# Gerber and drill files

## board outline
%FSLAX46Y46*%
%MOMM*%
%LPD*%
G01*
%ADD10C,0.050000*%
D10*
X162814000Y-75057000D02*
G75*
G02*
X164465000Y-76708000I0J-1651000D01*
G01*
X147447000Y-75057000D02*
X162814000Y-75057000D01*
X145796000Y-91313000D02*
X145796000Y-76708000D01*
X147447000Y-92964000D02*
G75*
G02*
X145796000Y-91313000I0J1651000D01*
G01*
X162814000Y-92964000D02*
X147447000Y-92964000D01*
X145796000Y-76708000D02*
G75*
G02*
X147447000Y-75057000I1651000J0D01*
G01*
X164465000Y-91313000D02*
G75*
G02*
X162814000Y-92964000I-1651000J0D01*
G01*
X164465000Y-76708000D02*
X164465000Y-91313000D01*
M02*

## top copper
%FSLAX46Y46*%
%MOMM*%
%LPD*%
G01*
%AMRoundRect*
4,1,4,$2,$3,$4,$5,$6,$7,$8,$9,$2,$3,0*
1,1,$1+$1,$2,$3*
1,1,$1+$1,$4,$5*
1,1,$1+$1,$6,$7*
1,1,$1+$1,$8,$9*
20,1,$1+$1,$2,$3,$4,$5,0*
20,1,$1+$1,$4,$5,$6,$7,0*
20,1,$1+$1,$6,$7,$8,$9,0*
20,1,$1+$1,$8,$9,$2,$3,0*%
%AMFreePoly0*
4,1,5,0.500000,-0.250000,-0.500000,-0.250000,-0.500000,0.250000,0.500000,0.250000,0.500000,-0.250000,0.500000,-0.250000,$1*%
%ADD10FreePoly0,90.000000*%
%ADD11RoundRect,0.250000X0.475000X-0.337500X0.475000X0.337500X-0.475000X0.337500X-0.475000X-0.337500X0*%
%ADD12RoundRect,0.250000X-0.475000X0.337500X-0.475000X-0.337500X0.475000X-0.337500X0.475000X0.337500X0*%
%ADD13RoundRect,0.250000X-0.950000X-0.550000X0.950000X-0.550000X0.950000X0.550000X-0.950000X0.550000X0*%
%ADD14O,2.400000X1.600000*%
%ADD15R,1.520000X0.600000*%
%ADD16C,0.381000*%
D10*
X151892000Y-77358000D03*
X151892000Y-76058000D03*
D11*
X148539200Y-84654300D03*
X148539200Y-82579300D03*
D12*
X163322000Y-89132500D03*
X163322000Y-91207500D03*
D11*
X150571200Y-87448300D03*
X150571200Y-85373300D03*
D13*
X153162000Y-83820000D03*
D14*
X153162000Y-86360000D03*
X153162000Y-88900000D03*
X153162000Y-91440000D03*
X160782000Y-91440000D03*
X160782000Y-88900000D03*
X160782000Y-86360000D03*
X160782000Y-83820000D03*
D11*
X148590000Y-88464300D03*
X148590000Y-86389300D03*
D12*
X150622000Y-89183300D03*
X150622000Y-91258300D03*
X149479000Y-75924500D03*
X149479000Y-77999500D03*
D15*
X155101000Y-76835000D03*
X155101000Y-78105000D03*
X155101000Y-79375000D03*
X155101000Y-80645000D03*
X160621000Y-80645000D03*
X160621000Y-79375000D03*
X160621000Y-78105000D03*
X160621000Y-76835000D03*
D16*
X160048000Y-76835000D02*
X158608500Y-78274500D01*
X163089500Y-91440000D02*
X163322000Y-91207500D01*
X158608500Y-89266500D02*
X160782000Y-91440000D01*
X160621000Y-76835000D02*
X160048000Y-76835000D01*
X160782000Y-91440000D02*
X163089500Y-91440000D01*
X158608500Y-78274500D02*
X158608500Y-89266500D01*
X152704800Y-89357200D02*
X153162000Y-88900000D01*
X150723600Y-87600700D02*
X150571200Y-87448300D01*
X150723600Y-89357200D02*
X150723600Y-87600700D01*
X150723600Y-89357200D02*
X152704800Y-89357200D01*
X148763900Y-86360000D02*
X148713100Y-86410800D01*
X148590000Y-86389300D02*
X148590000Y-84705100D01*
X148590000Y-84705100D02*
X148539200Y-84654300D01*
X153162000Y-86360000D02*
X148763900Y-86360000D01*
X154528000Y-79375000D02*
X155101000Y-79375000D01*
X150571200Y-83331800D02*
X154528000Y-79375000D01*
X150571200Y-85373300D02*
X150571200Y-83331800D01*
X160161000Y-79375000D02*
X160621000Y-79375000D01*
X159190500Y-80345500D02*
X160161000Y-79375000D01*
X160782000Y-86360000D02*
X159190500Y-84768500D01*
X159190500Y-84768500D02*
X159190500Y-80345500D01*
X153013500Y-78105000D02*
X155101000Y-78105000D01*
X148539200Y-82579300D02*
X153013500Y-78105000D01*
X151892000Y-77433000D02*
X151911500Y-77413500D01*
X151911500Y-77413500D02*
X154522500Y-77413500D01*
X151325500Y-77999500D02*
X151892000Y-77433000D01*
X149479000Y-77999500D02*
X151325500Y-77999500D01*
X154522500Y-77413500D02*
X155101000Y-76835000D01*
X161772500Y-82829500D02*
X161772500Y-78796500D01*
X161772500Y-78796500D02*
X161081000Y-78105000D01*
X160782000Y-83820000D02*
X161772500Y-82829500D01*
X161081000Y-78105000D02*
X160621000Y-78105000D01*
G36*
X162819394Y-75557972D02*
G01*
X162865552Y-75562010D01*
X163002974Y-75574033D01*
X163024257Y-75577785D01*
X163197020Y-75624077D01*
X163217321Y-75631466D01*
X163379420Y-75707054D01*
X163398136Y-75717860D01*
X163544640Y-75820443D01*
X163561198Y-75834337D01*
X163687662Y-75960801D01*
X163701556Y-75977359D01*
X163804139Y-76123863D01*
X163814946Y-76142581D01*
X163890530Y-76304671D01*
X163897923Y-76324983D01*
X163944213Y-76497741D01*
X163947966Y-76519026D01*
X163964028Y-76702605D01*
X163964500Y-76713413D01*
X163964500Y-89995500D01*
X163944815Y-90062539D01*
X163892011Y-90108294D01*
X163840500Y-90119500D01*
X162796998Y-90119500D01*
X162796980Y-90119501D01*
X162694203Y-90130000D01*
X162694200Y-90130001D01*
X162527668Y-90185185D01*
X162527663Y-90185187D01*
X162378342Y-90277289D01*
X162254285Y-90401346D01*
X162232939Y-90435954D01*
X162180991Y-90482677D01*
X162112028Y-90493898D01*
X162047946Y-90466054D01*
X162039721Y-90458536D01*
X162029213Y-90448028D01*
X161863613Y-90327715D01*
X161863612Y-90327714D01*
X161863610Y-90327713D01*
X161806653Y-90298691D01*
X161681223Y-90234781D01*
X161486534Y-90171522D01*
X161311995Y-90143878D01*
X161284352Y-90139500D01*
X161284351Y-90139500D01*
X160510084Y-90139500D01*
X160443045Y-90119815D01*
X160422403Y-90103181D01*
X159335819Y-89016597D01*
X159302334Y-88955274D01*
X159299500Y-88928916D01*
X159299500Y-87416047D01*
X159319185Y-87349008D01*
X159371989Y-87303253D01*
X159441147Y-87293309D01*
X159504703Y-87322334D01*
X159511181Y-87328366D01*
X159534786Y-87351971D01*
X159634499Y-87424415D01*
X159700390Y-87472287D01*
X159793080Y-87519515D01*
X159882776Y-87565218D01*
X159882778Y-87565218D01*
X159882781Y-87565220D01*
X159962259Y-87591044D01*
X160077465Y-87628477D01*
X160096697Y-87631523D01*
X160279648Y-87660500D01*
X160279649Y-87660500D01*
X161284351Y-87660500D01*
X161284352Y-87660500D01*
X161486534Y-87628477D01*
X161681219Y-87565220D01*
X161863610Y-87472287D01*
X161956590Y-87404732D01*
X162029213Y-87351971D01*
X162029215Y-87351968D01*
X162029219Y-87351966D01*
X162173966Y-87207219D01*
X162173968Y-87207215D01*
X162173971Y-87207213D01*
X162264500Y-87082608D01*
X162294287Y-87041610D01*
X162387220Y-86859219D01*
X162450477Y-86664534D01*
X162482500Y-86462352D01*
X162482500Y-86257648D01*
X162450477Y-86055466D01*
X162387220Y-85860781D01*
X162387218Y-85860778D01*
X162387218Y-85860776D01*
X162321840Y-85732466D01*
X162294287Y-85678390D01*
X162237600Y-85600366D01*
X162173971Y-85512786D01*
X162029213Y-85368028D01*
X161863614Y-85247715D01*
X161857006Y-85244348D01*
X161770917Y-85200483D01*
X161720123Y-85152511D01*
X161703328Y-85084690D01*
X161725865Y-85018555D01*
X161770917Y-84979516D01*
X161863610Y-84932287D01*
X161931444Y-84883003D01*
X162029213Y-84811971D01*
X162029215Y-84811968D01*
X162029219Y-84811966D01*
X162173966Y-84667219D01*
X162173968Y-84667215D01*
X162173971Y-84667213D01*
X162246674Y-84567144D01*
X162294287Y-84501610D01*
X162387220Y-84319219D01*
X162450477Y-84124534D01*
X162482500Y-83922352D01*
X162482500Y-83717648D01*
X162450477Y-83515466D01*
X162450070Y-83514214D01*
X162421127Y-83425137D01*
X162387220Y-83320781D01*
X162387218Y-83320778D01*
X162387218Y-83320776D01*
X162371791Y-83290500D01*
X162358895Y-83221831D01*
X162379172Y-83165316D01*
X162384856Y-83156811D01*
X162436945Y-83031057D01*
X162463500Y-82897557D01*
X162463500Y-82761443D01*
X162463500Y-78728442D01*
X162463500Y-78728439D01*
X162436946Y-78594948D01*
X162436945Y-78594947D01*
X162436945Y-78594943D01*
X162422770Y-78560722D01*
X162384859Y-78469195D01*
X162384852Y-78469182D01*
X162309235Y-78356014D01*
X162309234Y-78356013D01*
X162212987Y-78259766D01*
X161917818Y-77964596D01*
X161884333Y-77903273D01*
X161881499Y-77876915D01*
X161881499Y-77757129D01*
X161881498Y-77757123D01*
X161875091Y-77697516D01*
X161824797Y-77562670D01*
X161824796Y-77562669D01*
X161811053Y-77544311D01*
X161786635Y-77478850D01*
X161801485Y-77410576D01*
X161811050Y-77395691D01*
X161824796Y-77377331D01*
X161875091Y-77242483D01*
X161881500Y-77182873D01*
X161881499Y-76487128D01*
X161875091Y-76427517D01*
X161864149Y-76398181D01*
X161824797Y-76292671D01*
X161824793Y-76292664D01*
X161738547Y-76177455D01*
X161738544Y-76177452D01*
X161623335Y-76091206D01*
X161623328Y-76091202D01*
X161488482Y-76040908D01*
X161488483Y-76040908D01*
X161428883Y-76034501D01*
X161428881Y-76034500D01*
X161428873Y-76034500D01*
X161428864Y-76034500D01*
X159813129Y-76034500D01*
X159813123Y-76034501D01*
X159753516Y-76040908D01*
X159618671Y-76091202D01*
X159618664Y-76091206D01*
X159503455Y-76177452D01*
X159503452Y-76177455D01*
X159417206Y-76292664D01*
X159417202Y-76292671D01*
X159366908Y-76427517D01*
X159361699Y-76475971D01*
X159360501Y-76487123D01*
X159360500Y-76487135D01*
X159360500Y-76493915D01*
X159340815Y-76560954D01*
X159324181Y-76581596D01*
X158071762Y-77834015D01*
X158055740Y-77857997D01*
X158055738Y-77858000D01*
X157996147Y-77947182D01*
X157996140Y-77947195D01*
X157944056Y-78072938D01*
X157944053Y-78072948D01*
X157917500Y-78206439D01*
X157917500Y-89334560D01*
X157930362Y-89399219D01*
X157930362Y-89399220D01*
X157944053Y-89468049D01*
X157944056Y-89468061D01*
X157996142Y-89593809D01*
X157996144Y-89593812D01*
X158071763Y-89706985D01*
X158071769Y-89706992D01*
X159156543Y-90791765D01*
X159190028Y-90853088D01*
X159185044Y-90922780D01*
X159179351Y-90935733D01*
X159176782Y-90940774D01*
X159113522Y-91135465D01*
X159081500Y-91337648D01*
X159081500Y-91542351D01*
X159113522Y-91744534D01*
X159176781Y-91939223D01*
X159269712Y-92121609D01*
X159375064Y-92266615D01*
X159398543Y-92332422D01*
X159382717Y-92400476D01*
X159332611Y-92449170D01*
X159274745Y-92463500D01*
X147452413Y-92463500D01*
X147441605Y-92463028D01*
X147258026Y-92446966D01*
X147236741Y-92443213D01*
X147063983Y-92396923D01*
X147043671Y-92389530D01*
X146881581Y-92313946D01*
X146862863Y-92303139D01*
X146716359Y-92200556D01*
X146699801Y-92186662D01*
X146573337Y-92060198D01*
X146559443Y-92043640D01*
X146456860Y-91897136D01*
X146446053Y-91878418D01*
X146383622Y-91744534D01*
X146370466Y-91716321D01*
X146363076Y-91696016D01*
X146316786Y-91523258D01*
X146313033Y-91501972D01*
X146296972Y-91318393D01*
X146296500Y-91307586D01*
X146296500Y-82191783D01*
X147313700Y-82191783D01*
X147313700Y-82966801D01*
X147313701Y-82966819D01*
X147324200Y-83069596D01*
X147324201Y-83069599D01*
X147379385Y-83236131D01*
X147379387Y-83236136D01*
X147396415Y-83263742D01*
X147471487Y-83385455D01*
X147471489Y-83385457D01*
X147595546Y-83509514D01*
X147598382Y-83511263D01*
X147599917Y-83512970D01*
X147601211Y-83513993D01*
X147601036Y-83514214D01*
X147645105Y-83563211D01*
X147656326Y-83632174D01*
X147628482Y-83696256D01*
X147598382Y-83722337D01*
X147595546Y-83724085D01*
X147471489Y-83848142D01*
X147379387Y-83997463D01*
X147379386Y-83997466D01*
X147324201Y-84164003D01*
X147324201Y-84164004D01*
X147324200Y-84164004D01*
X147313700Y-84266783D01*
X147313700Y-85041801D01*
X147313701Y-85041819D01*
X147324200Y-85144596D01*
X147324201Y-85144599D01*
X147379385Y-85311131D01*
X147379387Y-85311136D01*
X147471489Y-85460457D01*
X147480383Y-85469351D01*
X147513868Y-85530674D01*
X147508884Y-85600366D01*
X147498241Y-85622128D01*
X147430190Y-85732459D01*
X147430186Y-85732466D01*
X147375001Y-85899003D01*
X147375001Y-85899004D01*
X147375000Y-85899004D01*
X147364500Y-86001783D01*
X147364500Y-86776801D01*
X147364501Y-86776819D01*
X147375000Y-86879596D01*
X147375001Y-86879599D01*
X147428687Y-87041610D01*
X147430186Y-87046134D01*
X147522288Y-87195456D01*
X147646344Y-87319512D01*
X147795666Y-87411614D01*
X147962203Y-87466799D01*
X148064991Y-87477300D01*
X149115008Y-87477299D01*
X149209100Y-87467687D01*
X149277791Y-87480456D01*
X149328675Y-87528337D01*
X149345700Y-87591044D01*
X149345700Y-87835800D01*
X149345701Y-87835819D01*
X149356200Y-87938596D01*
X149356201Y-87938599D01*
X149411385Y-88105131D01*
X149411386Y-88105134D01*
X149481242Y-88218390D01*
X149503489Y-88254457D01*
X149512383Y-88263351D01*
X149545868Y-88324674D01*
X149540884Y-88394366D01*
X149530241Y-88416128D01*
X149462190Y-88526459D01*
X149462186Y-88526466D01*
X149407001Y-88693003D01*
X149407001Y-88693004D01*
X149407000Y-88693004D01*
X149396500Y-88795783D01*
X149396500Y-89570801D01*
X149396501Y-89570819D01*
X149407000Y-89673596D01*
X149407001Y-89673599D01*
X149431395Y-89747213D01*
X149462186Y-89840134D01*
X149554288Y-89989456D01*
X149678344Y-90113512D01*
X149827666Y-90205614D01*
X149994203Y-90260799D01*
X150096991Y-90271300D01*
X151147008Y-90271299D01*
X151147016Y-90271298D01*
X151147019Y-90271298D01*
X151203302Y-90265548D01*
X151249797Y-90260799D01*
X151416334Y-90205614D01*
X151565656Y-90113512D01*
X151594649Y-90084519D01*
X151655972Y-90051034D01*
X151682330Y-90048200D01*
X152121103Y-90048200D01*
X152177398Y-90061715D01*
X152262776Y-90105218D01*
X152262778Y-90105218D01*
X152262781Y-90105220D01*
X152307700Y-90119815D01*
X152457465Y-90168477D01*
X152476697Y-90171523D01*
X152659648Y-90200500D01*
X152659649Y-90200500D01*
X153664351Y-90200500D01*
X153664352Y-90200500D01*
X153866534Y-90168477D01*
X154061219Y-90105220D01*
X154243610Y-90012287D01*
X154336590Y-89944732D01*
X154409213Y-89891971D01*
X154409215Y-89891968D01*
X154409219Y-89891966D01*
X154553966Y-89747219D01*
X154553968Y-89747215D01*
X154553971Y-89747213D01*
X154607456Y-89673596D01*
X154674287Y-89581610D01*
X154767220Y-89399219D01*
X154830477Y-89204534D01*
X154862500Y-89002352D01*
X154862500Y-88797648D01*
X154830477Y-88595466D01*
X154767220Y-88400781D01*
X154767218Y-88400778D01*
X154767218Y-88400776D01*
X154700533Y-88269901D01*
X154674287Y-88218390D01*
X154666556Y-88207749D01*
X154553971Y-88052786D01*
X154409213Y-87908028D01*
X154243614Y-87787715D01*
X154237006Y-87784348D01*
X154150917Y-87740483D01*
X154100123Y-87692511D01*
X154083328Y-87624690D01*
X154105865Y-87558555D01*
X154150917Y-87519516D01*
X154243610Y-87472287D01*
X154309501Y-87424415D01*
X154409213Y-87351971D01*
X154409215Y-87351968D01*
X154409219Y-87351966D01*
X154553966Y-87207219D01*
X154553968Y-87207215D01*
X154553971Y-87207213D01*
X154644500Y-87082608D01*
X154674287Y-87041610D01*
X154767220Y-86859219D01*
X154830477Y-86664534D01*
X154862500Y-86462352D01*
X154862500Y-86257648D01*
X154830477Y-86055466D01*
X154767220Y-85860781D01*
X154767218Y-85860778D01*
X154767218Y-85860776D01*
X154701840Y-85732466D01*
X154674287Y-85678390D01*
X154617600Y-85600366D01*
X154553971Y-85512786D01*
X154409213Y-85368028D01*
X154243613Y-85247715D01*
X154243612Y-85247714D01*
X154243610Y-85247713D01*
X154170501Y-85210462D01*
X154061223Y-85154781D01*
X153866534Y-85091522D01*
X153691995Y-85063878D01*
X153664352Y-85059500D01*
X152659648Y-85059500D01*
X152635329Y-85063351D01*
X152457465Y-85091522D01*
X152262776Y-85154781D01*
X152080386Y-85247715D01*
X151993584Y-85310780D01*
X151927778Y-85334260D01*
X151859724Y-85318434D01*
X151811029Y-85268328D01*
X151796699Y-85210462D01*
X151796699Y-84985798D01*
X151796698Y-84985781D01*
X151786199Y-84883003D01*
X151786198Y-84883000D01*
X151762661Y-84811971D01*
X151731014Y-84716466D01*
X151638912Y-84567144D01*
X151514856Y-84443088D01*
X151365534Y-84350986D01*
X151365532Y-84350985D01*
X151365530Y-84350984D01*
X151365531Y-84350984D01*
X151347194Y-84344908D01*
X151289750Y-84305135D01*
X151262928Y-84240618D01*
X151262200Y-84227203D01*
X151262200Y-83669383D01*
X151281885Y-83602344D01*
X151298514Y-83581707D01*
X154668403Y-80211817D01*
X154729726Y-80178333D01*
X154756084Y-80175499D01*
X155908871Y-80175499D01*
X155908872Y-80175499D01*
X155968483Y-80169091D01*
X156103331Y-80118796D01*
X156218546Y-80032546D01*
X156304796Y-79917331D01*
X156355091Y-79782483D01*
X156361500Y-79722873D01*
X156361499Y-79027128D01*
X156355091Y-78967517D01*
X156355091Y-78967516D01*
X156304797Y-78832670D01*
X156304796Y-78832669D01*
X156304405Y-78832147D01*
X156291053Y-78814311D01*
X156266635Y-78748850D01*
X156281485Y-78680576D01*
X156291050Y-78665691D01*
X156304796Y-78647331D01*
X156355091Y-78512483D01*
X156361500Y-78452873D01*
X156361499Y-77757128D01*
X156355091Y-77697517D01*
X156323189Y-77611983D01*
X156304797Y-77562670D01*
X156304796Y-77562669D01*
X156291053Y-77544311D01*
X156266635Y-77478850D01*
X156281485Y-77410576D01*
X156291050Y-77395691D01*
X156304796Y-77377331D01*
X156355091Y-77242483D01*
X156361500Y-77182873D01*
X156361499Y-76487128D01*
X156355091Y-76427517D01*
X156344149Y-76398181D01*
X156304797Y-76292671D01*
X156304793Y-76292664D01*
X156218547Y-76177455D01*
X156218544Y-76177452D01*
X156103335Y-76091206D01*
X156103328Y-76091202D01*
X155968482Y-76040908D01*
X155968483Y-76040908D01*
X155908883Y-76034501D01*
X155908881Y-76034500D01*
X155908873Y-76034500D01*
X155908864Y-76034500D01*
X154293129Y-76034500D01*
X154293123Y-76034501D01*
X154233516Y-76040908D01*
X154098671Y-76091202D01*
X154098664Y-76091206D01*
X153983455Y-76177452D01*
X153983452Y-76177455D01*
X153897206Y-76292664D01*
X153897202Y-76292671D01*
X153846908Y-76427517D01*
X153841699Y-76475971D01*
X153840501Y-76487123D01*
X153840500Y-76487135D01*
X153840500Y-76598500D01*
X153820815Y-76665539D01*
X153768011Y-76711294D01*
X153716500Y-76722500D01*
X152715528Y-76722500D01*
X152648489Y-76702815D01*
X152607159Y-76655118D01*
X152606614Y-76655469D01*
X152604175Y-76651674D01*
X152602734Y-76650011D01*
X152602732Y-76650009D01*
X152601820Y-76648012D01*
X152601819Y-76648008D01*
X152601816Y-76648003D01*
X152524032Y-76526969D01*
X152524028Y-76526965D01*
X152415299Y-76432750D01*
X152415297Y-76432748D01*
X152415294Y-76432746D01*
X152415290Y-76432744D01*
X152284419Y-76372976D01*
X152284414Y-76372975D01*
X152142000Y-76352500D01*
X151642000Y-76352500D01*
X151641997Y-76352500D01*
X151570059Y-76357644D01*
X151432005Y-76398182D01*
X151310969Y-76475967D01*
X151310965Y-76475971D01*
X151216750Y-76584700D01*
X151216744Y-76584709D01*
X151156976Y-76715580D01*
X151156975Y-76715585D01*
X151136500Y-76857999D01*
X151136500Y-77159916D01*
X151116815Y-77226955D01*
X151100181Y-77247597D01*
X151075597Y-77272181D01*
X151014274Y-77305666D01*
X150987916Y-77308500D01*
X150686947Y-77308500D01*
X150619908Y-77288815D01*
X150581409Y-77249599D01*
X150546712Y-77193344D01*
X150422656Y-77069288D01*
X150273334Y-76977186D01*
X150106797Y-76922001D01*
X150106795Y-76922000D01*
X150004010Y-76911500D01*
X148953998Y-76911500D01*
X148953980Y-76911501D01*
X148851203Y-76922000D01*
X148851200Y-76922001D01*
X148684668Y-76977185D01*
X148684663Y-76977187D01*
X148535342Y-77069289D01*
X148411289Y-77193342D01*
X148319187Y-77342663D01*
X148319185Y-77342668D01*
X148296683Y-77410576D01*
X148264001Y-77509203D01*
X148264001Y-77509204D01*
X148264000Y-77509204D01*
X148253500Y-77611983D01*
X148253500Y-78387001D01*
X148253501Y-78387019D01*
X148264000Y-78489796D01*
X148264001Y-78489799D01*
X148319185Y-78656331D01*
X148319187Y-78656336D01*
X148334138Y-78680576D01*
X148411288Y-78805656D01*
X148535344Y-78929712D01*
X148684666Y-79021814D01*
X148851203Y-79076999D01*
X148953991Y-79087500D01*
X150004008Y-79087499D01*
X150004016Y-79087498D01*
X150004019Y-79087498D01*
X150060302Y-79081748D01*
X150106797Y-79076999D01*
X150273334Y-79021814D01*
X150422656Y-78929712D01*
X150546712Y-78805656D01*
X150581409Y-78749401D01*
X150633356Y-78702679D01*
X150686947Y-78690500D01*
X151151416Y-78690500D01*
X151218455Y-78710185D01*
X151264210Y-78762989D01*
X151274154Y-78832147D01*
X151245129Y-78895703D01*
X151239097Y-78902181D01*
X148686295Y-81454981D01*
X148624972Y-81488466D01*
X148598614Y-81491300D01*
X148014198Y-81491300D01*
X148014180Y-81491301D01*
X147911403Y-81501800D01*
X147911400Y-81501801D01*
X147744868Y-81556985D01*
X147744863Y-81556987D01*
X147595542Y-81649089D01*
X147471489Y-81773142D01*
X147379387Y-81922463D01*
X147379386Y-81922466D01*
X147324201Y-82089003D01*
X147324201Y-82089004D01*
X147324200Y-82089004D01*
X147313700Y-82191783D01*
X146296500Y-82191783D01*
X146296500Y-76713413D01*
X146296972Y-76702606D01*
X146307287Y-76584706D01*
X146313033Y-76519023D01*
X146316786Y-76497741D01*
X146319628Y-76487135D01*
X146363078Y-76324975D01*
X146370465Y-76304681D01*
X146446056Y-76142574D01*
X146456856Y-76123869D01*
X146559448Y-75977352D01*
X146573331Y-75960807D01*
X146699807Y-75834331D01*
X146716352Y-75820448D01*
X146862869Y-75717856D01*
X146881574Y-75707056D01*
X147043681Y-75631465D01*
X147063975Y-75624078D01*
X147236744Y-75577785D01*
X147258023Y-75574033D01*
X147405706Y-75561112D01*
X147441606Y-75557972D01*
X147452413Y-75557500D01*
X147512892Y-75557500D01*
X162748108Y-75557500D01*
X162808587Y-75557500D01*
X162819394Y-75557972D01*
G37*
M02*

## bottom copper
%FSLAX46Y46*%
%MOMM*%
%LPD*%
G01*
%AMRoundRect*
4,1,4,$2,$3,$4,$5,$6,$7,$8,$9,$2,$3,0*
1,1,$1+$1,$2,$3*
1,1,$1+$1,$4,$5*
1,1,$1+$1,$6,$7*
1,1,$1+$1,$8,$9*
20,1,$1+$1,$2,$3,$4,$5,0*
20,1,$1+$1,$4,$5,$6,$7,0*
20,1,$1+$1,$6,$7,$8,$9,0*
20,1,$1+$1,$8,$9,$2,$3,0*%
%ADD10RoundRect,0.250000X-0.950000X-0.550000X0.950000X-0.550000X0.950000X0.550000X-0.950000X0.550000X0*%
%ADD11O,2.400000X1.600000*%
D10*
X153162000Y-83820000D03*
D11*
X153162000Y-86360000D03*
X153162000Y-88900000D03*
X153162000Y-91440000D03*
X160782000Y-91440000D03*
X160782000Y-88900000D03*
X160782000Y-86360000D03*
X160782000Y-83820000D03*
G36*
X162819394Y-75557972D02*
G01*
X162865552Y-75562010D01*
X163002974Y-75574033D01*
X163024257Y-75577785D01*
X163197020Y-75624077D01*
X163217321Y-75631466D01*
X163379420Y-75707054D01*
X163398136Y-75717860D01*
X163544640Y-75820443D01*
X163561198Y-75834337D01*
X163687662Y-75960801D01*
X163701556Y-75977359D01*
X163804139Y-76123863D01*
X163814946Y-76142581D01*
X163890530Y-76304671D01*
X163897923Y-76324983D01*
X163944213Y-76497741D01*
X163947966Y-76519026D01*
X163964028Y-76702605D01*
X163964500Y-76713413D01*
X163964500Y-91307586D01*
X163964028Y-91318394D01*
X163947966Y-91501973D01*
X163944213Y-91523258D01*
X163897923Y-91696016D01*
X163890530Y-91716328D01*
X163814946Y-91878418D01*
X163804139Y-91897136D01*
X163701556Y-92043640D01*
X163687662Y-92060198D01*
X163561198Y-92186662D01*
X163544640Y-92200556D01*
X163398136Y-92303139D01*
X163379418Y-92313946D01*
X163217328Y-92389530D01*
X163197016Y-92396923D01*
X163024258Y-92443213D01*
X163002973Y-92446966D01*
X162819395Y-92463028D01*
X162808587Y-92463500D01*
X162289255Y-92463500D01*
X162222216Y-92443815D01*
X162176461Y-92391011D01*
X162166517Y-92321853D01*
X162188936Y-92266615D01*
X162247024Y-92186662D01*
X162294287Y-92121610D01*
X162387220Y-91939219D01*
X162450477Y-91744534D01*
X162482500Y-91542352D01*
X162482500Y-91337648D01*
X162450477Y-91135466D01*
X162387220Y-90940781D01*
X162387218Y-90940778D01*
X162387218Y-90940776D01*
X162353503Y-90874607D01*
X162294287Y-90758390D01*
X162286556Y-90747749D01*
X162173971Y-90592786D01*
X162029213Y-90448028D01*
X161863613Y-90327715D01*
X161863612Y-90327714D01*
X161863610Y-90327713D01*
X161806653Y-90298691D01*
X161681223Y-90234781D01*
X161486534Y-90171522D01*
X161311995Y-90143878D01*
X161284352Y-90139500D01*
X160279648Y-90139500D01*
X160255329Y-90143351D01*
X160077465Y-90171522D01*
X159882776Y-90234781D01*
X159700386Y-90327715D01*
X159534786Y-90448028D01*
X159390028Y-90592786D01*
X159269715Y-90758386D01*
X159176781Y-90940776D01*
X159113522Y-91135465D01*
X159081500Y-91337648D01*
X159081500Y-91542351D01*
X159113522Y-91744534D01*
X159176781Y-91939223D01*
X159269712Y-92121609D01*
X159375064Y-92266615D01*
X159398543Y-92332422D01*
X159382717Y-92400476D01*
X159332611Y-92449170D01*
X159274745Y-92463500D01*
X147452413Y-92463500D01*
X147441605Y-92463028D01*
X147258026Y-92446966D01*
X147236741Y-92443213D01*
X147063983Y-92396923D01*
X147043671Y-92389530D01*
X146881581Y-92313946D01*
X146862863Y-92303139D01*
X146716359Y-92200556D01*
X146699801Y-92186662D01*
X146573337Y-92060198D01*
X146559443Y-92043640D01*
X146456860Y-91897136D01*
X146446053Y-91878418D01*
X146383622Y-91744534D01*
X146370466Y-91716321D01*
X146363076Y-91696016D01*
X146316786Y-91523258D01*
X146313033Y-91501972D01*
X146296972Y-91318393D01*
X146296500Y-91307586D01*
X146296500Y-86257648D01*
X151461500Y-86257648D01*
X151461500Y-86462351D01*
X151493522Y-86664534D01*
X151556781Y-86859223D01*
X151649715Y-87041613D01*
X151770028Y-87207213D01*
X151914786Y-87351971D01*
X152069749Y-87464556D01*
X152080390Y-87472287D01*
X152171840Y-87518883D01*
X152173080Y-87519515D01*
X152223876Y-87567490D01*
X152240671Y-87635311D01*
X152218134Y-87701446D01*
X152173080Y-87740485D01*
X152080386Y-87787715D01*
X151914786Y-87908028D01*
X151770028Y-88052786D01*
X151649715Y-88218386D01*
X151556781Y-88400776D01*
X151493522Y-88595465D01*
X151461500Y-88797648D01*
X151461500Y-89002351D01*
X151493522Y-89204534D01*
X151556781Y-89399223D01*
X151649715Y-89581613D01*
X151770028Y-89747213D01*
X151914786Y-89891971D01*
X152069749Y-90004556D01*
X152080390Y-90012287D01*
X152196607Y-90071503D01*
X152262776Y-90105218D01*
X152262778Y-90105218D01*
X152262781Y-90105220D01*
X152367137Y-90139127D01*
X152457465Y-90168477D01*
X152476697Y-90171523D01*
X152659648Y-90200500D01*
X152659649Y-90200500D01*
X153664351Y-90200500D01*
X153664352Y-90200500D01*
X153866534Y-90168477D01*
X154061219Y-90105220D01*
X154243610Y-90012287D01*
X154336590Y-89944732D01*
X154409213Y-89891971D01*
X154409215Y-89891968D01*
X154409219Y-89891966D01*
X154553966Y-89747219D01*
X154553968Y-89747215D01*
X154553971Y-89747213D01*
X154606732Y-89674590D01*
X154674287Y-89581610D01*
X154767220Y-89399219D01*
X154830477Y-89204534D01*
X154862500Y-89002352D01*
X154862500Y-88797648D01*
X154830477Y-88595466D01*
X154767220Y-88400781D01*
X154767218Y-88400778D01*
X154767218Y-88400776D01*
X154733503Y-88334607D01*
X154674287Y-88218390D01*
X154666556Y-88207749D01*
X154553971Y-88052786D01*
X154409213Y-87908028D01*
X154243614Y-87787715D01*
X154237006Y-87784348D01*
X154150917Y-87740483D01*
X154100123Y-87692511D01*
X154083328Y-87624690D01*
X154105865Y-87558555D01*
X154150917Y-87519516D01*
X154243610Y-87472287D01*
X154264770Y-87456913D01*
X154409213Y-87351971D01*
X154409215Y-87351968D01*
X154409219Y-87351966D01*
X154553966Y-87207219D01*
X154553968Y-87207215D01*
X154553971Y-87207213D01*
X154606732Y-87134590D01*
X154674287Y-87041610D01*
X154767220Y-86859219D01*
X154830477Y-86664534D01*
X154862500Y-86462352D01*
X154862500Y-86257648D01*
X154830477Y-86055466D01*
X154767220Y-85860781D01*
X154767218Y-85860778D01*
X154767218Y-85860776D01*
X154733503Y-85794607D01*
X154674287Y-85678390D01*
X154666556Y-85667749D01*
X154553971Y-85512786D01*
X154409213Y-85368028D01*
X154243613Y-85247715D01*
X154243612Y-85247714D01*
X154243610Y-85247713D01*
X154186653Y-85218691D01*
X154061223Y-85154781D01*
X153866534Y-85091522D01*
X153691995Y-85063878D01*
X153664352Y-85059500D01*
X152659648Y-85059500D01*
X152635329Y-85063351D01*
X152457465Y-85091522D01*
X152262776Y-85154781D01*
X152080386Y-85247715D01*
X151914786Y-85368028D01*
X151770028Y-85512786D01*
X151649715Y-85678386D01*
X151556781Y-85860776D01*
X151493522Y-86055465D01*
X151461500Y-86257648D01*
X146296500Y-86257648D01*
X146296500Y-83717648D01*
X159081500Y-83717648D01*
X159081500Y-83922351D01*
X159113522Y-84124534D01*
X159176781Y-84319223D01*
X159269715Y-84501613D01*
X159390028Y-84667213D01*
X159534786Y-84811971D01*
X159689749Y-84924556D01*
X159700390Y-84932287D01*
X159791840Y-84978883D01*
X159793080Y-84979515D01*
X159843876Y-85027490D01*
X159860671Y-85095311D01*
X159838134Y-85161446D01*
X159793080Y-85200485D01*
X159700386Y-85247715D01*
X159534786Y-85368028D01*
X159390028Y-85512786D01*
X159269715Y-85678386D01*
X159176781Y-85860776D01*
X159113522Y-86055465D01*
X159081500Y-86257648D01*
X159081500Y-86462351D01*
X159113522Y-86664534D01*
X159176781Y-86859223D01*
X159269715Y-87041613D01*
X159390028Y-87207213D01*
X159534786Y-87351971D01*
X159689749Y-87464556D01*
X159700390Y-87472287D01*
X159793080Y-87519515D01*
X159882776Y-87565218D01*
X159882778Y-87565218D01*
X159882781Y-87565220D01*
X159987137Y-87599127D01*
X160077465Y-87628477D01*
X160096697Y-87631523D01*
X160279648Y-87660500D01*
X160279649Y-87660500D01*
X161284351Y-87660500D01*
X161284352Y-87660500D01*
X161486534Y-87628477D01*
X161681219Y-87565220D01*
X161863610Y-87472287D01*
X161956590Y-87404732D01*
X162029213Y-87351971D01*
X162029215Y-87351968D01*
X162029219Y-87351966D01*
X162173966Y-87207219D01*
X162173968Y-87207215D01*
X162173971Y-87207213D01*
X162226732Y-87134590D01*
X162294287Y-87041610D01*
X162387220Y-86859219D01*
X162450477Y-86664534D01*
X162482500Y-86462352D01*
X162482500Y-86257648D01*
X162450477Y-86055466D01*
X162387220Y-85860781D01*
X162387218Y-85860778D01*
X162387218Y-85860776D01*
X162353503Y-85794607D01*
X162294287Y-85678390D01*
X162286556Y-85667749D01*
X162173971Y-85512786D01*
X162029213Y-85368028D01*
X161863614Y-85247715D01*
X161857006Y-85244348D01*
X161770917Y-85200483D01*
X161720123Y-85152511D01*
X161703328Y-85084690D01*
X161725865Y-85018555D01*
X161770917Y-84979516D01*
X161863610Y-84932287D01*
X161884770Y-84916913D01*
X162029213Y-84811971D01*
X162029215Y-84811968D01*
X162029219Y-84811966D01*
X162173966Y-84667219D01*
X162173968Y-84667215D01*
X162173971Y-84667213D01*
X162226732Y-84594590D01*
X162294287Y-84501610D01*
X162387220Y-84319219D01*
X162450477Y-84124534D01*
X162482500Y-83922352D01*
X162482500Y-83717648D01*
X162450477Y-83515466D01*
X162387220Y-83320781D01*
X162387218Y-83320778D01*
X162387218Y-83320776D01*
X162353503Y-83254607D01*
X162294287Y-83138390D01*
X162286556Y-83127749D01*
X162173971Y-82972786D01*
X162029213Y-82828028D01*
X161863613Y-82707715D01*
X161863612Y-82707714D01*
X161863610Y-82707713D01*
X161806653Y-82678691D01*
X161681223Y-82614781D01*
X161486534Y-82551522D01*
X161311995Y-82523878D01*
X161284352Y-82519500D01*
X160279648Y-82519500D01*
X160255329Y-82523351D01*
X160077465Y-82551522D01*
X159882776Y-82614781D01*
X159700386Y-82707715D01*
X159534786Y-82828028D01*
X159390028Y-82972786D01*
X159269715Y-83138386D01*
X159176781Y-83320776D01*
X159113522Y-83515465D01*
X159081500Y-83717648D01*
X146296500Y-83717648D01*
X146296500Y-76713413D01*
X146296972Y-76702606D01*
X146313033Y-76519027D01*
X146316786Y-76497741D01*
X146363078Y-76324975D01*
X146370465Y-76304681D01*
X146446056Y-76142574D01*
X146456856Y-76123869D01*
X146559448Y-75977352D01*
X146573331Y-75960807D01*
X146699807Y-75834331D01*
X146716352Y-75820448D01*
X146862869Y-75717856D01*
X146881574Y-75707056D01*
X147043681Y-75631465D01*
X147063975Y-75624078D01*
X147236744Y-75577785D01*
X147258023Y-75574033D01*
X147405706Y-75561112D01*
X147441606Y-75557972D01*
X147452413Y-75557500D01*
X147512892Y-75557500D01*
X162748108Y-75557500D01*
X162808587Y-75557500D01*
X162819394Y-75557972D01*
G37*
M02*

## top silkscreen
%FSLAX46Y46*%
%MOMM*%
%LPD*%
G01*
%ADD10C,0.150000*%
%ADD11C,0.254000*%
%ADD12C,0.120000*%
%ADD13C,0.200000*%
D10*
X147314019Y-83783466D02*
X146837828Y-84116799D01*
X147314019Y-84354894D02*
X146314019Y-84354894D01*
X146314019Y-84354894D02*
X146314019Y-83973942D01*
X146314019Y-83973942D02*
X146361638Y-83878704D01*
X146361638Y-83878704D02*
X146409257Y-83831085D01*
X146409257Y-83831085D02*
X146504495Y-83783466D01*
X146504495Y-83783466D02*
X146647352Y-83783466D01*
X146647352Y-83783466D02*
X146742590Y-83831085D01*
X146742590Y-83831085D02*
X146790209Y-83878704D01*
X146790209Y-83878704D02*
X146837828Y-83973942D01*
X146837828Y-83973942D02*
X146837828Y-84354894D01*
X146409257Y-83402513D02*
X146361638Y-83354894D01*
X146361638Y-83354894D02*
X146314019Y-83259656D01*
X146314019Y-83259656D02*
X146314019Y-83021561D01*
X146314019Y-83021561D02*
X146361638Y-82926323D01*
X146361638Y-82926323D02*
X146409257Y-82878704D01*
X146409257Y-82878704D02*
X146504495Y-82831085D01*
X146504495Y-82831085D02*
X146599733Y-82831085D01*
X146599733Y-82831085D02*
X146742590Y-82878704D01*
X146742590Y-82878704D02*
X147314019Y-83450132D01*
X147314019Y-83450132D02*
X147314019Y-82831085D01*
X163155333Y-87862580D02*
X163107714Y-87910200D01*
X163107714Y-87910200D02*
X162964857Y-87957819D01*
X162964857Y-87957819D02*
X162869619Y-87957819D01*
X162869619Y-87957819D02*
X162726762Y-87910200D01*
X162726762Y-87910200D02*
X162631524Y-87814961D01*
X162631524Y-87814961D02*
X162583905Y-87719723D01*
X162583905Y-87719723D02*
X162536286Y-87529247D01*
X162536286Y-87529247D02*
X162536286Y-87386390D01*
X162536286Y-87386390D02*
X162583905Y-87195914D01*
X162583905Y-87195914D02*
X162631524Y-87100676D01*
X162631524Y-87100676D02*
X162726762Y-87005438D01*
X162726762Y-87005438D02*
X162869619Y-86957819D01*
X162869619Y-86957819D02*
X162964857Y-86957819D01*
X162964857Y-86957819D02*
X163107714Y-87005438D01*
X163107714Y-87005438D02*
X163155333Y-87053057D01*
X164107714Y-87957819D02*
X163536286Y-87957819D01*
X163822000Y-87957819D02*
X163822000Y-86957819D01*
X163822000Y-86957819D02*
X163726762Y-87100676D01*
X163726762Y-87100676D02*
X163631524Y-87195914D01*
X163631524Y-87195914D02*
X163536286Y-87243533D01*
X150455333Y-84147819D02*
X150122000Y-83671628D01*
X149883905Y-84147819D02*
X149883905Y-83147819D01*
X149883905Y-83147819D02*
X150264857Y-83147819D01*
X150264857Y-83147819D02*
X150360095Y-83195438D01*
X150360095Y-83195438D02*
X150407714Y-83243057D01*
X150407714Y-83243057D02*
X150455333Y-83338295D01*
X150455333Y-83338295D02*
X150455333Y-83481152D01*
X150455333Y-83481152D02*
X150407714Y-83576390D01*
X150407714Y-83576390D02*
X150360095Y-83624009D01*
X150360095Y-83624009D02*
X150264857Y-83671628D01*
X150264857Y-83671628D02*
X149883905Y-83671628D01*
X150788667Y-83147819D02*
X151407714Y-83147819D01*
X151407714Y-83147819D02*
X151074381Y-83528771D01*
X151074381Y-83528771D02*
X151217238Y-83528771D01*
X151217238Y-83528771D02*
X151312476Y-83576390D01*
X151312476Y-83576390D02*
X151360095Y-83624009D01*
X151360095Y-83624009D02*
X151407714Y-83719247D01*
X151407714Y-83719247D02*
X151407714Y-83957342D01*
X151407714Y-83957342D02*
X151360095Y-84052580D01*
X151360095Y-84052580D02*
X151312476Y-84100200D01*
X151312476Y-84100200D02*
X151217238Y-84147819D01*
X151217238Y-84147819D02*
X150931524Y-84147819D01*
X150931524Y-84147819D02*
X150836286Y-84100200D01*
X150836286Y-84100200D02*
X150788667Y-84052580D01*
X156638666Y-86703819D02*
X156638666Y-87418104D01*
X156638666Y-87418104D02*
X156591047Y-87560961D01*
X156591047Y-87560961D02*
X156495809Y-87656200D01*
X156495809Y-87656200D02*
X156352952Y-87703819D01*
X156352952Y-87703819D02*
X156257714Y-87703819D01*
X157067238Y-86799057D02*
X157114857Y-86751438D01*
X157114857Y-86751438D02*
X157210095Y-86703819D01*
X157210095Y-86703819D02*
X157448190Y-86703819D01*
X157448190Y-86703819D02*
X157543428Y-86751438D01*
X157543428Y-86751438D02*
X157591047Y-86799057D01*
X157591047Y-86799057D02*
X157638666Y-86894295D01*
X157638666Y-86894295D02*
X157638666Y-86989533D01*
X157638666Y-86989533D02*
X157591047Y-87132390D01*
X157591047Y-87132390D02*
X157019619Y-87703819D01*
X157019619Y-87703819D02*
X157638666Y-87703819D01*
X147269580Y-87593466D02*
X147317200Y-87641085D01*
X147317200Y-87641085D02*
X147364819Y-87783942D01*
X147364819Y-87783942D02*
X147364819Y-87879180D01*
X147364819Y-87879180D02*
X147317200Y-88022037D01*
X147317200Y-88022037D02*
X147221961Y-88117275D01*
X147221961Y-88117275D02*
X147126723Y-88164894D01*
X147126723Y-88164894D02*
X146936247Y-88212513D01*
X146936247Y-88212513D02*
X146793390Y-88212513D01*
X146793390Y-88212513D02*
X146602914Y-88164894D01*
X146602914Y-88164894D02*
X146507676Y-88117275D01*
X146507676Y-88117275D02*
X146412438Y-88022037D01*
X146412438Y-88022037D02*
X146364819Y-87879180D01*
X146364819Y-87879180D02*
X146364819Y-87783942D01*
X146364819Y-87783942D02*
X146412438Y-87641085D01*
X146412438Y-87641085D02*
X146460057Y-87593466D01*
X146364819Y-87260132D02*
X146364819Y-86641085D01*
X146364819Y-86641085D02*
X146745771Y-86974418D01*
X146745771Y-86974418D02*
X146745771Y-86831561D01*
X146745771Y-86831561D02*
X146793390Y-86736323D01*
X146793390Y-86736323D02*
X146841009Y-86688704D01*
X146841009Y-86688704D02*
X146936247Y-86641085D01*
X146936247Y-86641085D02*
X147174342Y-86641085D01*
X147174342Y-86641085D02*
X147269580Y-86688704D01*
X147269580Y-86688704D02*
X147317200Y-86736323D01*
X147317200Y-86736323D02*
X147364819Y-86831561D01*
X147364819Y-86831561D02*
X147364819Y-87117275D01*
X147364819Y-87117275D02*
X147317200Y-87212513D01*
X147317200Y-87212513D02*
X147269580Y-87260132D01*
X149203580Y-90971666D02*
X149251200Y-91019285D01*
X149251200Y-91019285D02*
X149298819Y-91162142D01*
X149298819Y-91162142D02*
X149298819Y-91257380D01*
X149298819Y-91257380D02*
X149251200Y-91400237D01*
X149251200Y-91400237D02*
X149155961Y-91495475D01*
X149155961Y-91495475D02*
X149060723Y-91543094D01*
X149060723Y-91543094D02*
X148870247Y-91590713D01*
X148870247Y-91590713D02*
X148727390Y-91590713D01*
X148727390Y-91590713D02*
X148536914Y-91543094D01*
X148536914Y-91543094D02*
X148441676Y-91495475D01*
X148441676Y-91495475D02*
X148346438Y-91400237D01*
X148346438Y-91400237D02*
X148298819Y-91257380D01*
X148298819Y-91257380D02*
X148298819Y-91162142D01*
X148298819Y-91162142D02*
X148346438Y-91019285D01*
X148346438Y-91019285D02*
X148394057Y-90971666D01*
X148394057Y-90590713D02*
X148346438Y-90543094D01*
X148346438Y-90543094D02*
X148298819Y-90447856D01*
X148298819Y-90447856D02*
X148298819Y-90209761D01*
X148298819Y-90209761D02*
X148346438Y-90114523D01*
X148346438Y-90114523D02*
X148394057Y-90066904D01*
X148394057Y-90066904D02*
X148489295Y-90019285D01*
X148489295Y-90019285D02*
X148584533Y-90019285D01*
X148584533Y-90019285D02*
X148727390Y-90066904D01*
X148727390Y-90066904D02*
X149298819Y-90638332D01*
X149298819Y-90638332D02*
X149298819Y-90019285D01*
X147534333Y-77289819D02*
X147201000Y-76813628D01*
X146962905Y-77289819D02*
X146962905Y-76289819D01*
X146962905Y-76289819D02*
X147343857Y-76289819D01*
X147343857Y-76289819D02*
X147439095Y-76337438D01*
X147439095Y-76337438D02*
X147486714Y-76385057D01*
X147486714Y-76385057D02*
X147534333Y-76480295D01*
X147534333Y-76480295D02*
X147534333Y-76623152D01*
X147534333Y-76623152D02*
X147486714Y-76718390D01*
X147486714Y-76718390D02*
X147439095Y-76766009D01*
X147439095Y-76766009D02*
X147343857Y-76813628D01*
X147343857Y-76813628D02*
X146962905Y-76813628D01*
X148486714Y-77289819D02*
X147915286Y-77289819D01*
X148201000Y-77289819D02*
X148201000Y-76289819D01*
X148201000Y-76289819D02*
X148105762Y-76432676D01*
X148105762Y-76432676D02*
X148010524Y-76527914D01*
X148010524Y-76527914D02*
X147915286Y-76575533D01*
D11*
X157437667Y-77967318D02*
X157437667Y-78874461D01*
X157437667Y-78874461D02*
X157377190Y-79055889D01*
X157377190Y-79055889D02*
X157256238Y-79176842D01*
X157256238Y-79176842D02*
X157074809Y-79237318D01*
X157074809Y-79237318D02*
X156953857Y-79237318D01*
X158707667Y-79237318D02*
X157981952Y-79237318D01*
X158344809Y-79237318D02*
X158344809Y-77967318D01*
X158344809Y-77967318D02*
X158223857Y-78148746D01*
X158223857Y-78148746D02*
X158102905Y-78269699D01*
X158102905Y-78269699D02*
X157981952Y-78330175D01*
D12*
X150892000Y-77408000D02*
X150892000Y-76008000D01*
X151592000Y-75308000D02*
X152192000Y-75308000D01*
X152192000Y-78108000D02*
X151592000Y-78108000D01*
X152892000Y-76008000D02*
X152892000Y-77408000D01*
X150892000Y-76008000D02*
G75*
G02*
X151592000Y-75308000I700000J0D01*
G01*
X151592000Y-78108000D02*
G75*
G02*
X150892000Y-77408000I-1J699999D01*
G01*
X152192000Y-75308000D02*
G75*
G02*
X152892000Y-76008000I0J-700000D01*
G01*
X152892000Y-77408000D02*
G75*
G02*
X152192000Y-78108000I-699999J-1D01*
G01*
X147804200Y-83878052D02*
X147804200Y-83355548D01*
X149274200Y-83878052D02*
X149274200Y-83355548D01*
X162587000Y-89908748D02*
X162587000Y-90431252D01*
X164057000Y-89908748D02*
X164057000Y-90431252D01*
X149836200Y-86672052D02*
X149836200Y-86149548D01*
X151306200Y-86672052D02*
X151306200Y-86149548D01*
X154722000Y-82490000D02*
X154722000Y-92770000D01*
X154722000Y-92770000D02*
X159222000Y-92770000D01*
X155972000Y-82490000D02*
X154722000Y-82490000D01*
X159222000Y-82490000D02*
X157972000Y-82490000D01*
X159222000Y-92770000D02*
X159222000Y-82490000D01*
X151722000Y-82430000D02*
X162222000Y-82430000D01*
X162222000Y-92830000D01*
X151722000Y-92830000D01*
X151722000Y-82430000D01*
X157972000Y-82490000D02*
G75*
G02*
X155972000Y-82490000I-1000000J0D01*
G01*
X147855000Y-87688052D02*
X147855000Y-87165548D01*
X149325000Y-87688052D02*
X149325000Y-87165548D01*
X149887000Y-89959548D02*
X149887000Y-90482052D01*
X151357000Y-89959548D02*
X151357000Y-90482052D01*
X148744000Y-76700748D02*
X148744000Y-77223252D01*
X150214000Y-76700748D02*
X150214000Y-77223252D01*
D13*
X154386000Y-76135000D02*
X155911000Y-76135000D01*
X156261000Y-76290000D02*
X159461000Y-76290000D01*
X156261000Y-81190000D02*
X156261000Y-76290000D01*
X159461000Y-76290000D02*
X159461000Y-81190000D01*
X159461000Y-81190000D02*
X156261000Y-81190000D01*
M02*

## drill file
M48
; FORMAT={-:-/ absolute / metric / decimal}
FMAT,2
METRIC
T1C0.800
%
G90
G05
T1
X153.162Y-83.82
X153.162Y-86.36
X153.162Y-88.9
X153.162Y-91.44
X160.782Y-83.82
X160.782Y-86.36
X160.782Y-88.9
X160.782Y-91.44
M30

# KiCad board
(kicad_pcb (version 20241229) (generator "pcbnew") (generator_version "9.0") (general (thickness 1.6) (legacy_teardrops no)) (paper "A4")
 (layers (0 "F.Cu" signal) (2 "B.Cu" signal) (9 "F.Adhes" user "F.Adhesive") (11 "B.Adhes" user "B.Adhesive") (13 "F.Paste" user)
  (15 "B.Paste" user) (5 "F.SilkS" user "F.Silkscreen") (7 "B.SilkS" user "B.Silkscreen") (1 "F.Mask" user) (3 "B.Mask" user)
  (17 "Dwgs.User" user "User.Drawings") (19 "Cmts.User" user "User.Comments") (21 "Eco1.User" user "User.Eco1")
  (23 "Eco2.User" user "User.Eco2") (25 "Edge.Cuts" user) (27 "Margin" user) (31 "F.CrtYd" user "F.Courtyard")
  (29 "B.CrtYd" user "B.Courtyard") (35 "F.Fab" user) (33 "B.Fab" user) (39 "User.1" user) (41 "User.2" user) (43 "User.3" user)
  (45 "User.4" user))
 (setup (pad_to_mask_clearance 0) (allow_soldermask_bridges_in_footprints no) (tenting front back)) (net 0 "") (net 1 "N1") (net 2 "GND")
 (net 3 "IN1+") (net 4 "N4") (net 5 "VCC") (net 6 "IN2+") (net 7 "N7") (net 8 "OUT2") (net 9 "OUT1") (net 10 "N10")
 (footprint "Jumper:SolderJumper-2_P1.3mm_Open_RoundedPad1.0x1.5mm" (layer "F.Cu") (at 151.892 76.708 90)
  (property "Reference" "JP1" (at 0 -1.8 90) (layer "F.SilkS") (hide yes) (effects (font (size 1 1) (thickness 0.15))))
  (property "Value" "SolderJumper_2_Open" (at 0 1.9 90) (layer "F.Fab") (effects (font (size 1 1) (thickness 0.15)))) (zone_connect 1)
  (fp_line (start -0.7 -1) (end 0.7 -1) (stroke (width 0.12) (type solid)) (layer "F.SilkS"))
  (fp_line (start 1.4 -0.3) (end 1.4 0.3) (stroke (width 0.12) (type solid)) (layer "F.SilkS"))
  (fp_line (start -1.4 0.3) (end -1.4 -0.3) (stroke (width 0.12) (type solid)) (layer "F.SilkS"))
  (fp_line (start 0.7 1) (end -0.7 1) (stroke (width 0.12) (type solid)) (layer "F.SilkS"))
  (fp_arc (start 0.7 -1) (mid 1.194975 -0.794975) (end 1.4 -0.3) (stroke (width 0.12) (type solid)) (layer "F.SilkS"))
  (fp_arc (start -1.4 -0.3) (mid -1.194975 -0.794975) (end -0.7 -1) (stroke (width 0.12) (type solid)) (layer "F.SilkS"))
  (fp_arc (start 1.4 0.3) (mid 1.194975 0.794975) (end 0.7 1) (stroke (width 0.12) (type solid)) (layer "F.SilkS"))
  (fp_arc (start -0.7 1) (mid -1.194975 0.794975) (end -1.4 0.3) (stroke (width 0.12) (type solid)) (layer "F.SilkS"))
  (pad "1" smd custom (at -0.65 0 90) (size 1 0.5) (layers "F.Cu" "F.Mask") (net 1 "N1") (zone_connect 2) (thermal_bridge_angle 45)
   (options (clearance outline) (anchor rect)) (primitives))
  (pad "2" smd custom (at 0.65 0 90) (size 1 0.5) (layers "F.Cu" "F.Mask") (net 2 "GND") (zone_connect 2) (thermal_bridge_angle 45)
   (options (clearance outline) (anchor rect)) (primitives)))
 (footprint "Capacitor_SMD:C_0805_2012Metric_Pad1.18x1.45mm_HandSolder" (layer "F.Cu") (at 148.5392 83.6168 90)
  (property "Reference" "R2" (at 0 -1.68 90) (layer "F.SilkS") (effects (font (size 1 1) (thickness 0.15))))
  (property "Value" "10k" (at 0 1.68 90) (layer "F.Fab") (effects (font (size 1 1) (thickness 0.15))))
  (fp_line (start -0.261252 -0.735) (end 0.261252 -0.735) (stroke (width 0.12) (type solid)) (layer "F.SilkS"))
  (fp_line (start -0.261252 0.735) (end 0.261252 0.735) (stroke (width 0.12) (type solid)) (layer "F.SilkS"))
  (pad "1" smd roundrect (at -1.0375 0 90) (size 1.175 1.45) (layers "F.Cu" "F.Mask" "F.Paste") (roundrect_rratio 0.212766) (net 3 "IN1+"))
  (pad "2" smd roundrect (at 1.0375 0 90) (size 1.175 1.45) (layers "F.Cu" "F.Mask" "F.Paste") (roundrect_rratio 0.212766) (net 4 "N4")))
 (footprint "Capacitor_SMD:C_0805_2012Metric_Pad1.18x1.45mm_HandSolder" (layer "F.Cu") (at 163.322 90.17 -90)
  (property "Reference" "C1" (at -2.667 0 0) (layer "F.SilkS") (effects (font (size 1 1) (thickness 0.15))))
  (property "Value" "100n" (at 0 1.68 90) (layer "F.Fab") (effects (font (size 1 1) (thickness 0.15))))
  (fp_line (start -0.261252 0.735) (end 0.261252 0.735) (stroke (width 0.12) (type solid)) (layer "F.SilkS"))
  (fp_line (start -0.261252 -0.735) (end 0.261252 -0.735) (stroke (width 0.12) (type solid)) (layer "F.SilkS"))
  (pad "1" smd roundrect (at -1.0375 0 270) (size 1.175 1.45) (layers "F.Cu" "F.Mask" "F.Paste") (roundrect_rratio 0.212766) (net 2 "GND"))
  (pad "2" smd roundrect (at 1.0375 0 270) (size 1.175 1.45) (layers "F.Cu" "F.Mask" "F.Paste") (roundrect_rratio 0.212766) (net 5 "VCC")))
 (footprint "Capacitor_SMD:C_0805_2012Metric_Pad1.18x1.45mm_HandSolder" (layer "F.Cu") (at 150.5712 86.4108 90)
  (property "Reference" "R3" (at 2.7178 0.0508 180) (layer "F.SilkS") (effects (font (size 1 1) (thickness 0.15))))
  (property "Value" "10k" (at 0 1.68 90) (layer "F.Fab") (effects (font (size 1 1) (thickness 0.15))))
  (fp_line (start -0.261252 -0.735) (end 0.261252 -0.735) (stroke (width 0.12) (type solid)) (layer "F.SilkS"))
  (fp_line (start -0.261252 0.735) (end 0.261252 0.735) (stroke (width 0.12) (type solid)) (layer "F.SilkS"))
  (pad "1" smd roundrect (at -1.0375 0 90) (size 1.175 1.45) (layers "F.Cu" "F.Mask" "F.Paste") (roundrect_rratio 0.212766) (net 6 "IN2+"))
  (pad "2" smd roundrect (at 1.0375 0 90) (size 1.175 1.45) (layers "F.Cu" "F.Mask" "F.Paste") (roundrect_rratio 0.212766) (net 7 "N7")))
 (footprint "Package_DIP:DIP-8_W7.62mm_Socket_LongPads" (layer "F.Cu") (at 153.162 83.82)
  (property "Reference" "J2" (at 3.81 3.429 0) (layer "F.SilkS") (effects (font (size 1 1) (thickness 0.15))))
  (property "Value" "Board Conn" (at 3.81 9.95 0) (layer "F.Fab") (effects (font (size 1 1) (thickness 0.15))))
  (fp_line (start 1.56 -1.33) (end 1.56 8.95) (stroke (width 0.12) (type solid)) (layer "F.SilkS"))
  (fp_line (start 1.56 8.95) (end 6.06 8.95) (stroke (width 0.12) (type solid)) (layer "F.SilkS"))
  (fp_line (start 2.81 -1.33) (end 1.56 -1.33) (stroke (width 0.12) (type solid)) (layer "F.SilkS"))
  (fp_line (start 6.06 -1.33) (end 4.81 -1.33) (stroke (width 0.12) (type solid)) (layer "F.SilkS"))
  (fp_line (start 6.06 8.95) (end 6.06 -1.33) (stroke (width 0.12) (type solid)) (layer "F.SilkS"))
  (fp_rect (start -1.44 -1.39) (end 9.06 9.01) (stroke (width 0.12) (type solid)) (fill no) (layer "F.SilkS"))
  (fp_arc (start 4.81 -1.33) (mid 3.81 -0.33) (end 2.81 -1.33) (stroke (width 0.12) (type solid)) (layer "F.SilkS"))
  (pad "1" thru_hole roundrect (at 0 0) (size 2.4 1.6) (drill 0.8) (layers "*.Cu" "*.Mask") (remove_unused_layers no)
   (roundrect_rratio 0.15625) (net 2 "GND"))
  (pad "2" thru_hole oval (at 0 2.54) (size 2.4 1.6) (drill 0.8) (layers "*.Cu" "*.Mask") (remove_unused_layers no) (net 3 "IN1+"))
  (pad "3" thru_hole oval (at 0 5.08) (size 2.4 1.6) (drill 0.8) (layers "*.Cu" "*.Mask") (remove_unused_layers no) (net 6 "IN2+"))
  (pad "4" thru_hole oval (at 0 7.62) (size 2.4 1.6) (drill 0.8) (layers "*.Cu" "*.Mask") (remove_unused_layers no) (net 2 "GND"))
  (pad "5" thru_hole oval (at 7.62 7.62) (size 2.4 1.6) (drill 0.8) (layers "*.Cu" "*.Mask") (remove_unused_layers no) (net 5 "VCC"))
  (pad "6" thru_hole oval (at 7.62 5.08) (size 2.4 1.6) (drill 0.8) (layers "*.Cu" "*.Mask") (remove_unused_layers no) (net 2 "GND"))
  (pad "7" thru_hole oval (at 7.62 2.54) (size 2.4 1.6) (drill 0.8) (layers "*.Cu" "*.Mask") (remove_unused_layers no) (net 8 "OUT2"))
  (pad "8" thru_hole oval (at 7.62 0) (size 2.4 1.6) (drill 0.8) (layers "*.Cu" "*.Mask") (remove_unused_layers no) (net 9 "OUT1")))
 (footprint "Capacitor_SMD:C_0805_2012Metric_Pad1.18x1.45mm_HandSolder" (layer "F.Cu") (at 148.59 87.4268 90)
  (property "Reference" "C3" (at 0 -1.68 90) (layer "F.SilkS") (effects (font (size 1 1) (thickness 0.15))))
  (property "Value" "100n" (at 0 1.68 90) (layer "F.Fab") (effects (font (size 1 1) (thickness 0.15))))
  (fp_line (start -0.261252 -0.735) (end 0.261252 -0.735) (stroke (width 0.12) (type solid)) (layer "F.SilkS"))
  (fp_line (start -0.261252 0.735) (end 0.261252 0.735) (stroke (width 0.12) (type solid)) (layer "F.SilkS"))
  (pad "1" smd roundrect (at -1.0375 0 90) (size 1.175 1.45) (layers "F.Cu" "F.Mask" "F.Paste") (roundrect_rratio 0.212766) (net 2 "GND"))
  (pad "2" smd roundrect (at 1.0375 0 90) (size 1.175 1.45) (layers "F.Cu" "F.Mask" "F.Paste") (roundrect_rratio 0.212766) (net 3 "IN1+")))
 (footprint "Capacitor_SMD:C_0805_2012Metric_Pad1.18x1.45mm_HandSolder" (layer "F.Cu") (at 150.622 90.2208 -90)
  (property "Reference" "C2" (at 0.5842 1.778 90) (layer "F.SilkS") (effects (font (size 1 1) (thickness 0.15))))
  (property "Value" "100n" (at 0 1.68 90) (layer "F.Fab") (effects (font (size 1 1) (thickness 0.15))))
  (fp_line (start -0.261252 0.735) (end 0.261252 0.735) (stroke (width 0.12) (type solid)) (layer "F.SilkS"))
  (fp_line (start -0.261252 -0.735) (end 0.261252 -0.735) (stroke (width 0.12) (type solid)) (layer "F.SilkS"))
  (pad "1" smd roundrect (at -1.0375 0 270) (size 1.175 1.45) (layers "F.Cu" "F.Mask" "F.Paste") (roundrect_rratio 0.212766) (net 6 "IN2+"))
  (pad "2" smd roundrect (at 1.0375 0 270) (size 1.175 1.45) (layers "F.Cu" "F.Mask" "F.Paste") (roundrect_rratio 0.212766) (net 2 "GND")))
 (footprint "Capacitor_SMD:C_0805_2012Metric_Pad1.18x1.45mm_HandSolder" (layer "F.Cu") (at 149.479 76.962 -90)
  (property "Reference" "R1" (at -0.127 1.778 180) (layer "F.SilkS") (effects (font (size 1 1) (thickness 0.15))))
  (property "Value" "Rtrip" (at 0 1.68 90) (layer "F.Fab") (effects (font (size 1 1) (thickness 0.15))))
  (fp_line (start -0.261252 0.735) (end 0.261252 0.735) (stroke (width 0.12) (type solid)) (layer "F.SilkS"))
  (fp_line (start -0.261252 -0.735) (end 0.261252 -0.735) (stroke (width 0.12) (type solid)) (layer "F.SilkS"))
  (pad "1" smd roundrect (at -1.0375 0 270) (size 1.175 1.45) (layers "F.Cu" "F.Mask" "F.Paste") (roundrect_rratio 0.212766) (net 2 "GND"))
  (pad "2" smd roundrect (at 1.0375 0 270) (size 1.175 1.45) (layers "F.Cu" "F.Mask" "F.Paste") (roundrect_rratio 0.212766) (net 1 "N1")))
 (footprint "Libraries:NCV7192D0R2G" (layer "F.Cu") (at 157.861 78.74)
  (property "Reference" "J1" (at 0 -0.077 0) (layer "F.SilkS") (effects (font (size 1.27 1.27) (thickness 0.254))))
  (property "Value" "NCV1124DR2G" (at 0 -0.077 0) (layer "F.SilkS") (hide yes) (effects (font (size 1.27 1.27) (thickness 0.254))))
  (fp_line (start -3.475 -2.605) (end -1.95 -2.605) (stroke (width 0.2) (type solid)) (layer "F.SilkS"))
  (fp_line (start -1.6 -2.45) (end 1.6 -2.45) (stroke (width 0.2) (type solid)) (layer "F.SilkS"))
  (fp_line (start -1.6 2.45) (end -1.6 -2.45) (stroke (width 0.2) (type solid)) (layer "F.SilkS"))
  (fp_line (start 1.6 -2.45) (end 1.6 2.45) (stroke (width 0.2) (type solid)) (layer "F.SilkS"))
  (fp_line (start 1.6 2.45) (end -1.6 2.45) (stroke (width 0.2) (type solid)) (layer "F.SilkS"))
  (pad "1" smd rect (at -2.76 -1.905 90) (size 0.6 1.52) (layers "F.Cu" "F.Mask" "F.Paste") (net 1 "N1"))
  (pad "2" smd rect (at -2.76 -0.635 90) (size 0.6 1.52) (layers "F.Cu" "F.Mask" "F.Paste") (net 4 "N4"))
  (pad "3" smd rect (at -2.76 0.635 90) (size 0.6 1.52) (layers "F.Cu" "F.Mask" "F.Paste") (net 7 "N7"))
  (pad "4" smd rect (at -2.76 1.905 90) (size 0.6 1.52) (layers "F.Cu" "F.Mask" "F.Paste") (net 2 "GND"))
  (pad "5" smd rect (at 2.76 1.905 90) (size 0.6 1.52) (layers "F.Cu" "F.Mask" "F.Paste") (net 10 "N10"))
  (pad "6" smd rect (at 2.76 0.635 90) (size 0.6 1.52) (layers "F.Cu" "F.Mask" "F.Paste") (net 8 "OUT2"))
  (pad "7" smd rect (at 2.76 -0.635 90) (size 0.6 1.52) (layers "F.Cu" "F.Mask" "F.Paste") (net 9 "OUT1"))
  (pad "8" smd rect (at 2.76 -1.905 90) (size 0.6 1.52) (layers "F.Cu" "F.Mask" "F.Paste") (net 5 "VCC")))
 (gr_arc (start 162.814 75.057) (mid 163.981433 75.540567) (end 164.465 76.708) (stroke (width 0.05) (type default)) (layer "Edge.Cuts"))
 (gr_line (start 147.447 75.057) (end 162.814 75.057) (stroke (width 0.05) (type default)) (layer "Edge.Cuts"))
 (gr_line (start 145.796 91.313) (end 145.796 76.708) (stroke (width 0.05) (type default)) (layer "Edge.Cuts"))
 (gr_arc (start 147.447 92.964) (mid 146.279567 92.480433) (end 145.796 91.313) (stroke (width 0.05) (type default)) (layer "Edge.Cuts"))
 (gr_line (start 162.814 92.964) (end 147.447 92.964) (stroke (width 0.05) (type default)) (layer "Edge.Cuts"))
 (gr_arc (start 145.796 76.708) (mid 146.279567 75.540567) (end 147.447 75.057) (stroke (width 0.05) (type default)) (layer "Edge.Cuts"))
 (gr_arc (start 164.465 91.313) (mid 163.981433 92.480433) (end 162.814 92.964) (stroke (width 0.05) (type default)) (layer "Edge.Cuts"))
 (gr_line (start 164.465 76.708) (end 164.465 91.313) (stroke (width 0.05) (type default)) (layer "Edge.Cuts"))
 (segment (start 160.048 76.835) (end 158.6085 78.2745) (width 0.381) (layer "F.Cu") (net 5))
 (segment (start 163.0895 91.44) (end 163.322 91.2075) (width 0.381) (layer "F.Cu") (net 5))
 (segment (start 158.6085 89.2665) (end 160.782 91.44) (width 0.381) (layer "F.Cu") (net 5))
 (segment (start 160.621 76.835) (end 160.048 76.835) (width 0.381) (layer "F.Cu") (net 5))
 (segment (start 160.782 91.44) (end 163.0895 91.44) (width 0.381) (layer "F.Cu") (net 5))
 (segment (start 158.6085 78.2745) (end 158.6085 89.2665) (width 0.381) (layer "F.Cu") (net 5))
 (segment (start 152.7048 89.3572) (end 153.162 88.9) (width 0.381) (layer "F.Cu") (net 6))
 (segment (start 150.7236 87.6007) (end 150.5712 87.4483) (width 0.381) (layer "F.Cu") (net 6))
 (segment (start 150.7236 89.3572) (end 150.7236 87.6007) (width 0.381) (layer "F.Cu") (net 6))
 (segment (start 150.7236 89.3572) (end 152.7048 89.3572) (width 0.381) (layer "F.Cu") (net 6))
 (segment (start 148.7639 86.36) (end 148.7131 86.4108) (width 0.381) (layer "F.Cu") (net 3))
 (segment (start 148.59 86.3893) (end 148.59 84.7051) (width 0.381) (layer "F.Cu") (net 3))
 (segment (start 148.59 84.7051) (end 148.5392 84.6543) (width 0.381) (layer "F.Cu") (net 3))
 (segment (start 153.162 86.36) (end 148.7639 86.36) (width 0.381) (layer "F.Cu") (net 3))
 (segment (start 154.528 79.375) (end 155.101 79.375) (width 0.381) (layer "F.Cu") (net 7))
 (segment (start 150.5712 83.3318) (end 154.528 79.375) (width 0.381) (layer "F.Cu") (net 7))
 (segment (start 150.5712 85.3733) (end 150.5712 83.3318) (width 0.381) (layer "F.Cu") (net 7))
 (segment (start 160.161 79.375) (end 160.621 79.375) (width 0.381) (layer "F.Cu") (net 8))
 (segment (start 159.1905 80.3455) (end 160.161 79.375) (width 0.381) (layer "F.Cu") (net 8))
 (segment (start 160.782 86.36) (end 159.1905 84.7685) (width 0.381) (layer "F.Cu") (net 8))
 (segment (start 159.1905 84.7685) (end 159.1905 80.3455) (width 0.381) (layer "F.Cu") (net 8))
 (segment (start 153.0135 78.105) (end 155.101 78.105) (width 0.381) (layer "F.Cu") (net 4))
 (segment (start 148.5392 82.5793) (end 153.0135 78.105) (width 0.381) (layer "F.Cu") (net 4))
 (segment (start 151.892 77.433) (end 151.9115 77.4135) (width 0.381) (layer "F.Cu") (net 1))
 (segment (start 151.9115 77.4135) (end 154.5225 77.4135) (width 0.381) (layer "F.Cu") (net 1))
 (segment (start 151.3255 77.9995) (end 151.892 77.433) (width 0.381) (layer "F.Cu") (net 1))
 (segment (start 149.479 77.9995) (end 151.3255 77.9995) (width 0.381) (layer "F.Cu") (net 1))
 (segment (start 154.5225 77.4135) (end 155.101 76.835) (width 0.381) (layer "F.Cu") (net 1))
 (segment (start 161.7725 82.8295) (end 161.7725 78.7965) (width 0.381) (layer "F.Cu") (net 9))
 (segment (start 161.7725 78.7965) (end 161.081 78.105) (width 0.381) (layer "F.Cu") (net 9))
 (segment (start 160.782 83.82) (end 161.7725 82.8295) (width 0.381) (layer "F.Cu") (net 9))
 (segment (start 161.081 78.105) (end 160.621 78.105) (width 0.381) (layer "F.Cu") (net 9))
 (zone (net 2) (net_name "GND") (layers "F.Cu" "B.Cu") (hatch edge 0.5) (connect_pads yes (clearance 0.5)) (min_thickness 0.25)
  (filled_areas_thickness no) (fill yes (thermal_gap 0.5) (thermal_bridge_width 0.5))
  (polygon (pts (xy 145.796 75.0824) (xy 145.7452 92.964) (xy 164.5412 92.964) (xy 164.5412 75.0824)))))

